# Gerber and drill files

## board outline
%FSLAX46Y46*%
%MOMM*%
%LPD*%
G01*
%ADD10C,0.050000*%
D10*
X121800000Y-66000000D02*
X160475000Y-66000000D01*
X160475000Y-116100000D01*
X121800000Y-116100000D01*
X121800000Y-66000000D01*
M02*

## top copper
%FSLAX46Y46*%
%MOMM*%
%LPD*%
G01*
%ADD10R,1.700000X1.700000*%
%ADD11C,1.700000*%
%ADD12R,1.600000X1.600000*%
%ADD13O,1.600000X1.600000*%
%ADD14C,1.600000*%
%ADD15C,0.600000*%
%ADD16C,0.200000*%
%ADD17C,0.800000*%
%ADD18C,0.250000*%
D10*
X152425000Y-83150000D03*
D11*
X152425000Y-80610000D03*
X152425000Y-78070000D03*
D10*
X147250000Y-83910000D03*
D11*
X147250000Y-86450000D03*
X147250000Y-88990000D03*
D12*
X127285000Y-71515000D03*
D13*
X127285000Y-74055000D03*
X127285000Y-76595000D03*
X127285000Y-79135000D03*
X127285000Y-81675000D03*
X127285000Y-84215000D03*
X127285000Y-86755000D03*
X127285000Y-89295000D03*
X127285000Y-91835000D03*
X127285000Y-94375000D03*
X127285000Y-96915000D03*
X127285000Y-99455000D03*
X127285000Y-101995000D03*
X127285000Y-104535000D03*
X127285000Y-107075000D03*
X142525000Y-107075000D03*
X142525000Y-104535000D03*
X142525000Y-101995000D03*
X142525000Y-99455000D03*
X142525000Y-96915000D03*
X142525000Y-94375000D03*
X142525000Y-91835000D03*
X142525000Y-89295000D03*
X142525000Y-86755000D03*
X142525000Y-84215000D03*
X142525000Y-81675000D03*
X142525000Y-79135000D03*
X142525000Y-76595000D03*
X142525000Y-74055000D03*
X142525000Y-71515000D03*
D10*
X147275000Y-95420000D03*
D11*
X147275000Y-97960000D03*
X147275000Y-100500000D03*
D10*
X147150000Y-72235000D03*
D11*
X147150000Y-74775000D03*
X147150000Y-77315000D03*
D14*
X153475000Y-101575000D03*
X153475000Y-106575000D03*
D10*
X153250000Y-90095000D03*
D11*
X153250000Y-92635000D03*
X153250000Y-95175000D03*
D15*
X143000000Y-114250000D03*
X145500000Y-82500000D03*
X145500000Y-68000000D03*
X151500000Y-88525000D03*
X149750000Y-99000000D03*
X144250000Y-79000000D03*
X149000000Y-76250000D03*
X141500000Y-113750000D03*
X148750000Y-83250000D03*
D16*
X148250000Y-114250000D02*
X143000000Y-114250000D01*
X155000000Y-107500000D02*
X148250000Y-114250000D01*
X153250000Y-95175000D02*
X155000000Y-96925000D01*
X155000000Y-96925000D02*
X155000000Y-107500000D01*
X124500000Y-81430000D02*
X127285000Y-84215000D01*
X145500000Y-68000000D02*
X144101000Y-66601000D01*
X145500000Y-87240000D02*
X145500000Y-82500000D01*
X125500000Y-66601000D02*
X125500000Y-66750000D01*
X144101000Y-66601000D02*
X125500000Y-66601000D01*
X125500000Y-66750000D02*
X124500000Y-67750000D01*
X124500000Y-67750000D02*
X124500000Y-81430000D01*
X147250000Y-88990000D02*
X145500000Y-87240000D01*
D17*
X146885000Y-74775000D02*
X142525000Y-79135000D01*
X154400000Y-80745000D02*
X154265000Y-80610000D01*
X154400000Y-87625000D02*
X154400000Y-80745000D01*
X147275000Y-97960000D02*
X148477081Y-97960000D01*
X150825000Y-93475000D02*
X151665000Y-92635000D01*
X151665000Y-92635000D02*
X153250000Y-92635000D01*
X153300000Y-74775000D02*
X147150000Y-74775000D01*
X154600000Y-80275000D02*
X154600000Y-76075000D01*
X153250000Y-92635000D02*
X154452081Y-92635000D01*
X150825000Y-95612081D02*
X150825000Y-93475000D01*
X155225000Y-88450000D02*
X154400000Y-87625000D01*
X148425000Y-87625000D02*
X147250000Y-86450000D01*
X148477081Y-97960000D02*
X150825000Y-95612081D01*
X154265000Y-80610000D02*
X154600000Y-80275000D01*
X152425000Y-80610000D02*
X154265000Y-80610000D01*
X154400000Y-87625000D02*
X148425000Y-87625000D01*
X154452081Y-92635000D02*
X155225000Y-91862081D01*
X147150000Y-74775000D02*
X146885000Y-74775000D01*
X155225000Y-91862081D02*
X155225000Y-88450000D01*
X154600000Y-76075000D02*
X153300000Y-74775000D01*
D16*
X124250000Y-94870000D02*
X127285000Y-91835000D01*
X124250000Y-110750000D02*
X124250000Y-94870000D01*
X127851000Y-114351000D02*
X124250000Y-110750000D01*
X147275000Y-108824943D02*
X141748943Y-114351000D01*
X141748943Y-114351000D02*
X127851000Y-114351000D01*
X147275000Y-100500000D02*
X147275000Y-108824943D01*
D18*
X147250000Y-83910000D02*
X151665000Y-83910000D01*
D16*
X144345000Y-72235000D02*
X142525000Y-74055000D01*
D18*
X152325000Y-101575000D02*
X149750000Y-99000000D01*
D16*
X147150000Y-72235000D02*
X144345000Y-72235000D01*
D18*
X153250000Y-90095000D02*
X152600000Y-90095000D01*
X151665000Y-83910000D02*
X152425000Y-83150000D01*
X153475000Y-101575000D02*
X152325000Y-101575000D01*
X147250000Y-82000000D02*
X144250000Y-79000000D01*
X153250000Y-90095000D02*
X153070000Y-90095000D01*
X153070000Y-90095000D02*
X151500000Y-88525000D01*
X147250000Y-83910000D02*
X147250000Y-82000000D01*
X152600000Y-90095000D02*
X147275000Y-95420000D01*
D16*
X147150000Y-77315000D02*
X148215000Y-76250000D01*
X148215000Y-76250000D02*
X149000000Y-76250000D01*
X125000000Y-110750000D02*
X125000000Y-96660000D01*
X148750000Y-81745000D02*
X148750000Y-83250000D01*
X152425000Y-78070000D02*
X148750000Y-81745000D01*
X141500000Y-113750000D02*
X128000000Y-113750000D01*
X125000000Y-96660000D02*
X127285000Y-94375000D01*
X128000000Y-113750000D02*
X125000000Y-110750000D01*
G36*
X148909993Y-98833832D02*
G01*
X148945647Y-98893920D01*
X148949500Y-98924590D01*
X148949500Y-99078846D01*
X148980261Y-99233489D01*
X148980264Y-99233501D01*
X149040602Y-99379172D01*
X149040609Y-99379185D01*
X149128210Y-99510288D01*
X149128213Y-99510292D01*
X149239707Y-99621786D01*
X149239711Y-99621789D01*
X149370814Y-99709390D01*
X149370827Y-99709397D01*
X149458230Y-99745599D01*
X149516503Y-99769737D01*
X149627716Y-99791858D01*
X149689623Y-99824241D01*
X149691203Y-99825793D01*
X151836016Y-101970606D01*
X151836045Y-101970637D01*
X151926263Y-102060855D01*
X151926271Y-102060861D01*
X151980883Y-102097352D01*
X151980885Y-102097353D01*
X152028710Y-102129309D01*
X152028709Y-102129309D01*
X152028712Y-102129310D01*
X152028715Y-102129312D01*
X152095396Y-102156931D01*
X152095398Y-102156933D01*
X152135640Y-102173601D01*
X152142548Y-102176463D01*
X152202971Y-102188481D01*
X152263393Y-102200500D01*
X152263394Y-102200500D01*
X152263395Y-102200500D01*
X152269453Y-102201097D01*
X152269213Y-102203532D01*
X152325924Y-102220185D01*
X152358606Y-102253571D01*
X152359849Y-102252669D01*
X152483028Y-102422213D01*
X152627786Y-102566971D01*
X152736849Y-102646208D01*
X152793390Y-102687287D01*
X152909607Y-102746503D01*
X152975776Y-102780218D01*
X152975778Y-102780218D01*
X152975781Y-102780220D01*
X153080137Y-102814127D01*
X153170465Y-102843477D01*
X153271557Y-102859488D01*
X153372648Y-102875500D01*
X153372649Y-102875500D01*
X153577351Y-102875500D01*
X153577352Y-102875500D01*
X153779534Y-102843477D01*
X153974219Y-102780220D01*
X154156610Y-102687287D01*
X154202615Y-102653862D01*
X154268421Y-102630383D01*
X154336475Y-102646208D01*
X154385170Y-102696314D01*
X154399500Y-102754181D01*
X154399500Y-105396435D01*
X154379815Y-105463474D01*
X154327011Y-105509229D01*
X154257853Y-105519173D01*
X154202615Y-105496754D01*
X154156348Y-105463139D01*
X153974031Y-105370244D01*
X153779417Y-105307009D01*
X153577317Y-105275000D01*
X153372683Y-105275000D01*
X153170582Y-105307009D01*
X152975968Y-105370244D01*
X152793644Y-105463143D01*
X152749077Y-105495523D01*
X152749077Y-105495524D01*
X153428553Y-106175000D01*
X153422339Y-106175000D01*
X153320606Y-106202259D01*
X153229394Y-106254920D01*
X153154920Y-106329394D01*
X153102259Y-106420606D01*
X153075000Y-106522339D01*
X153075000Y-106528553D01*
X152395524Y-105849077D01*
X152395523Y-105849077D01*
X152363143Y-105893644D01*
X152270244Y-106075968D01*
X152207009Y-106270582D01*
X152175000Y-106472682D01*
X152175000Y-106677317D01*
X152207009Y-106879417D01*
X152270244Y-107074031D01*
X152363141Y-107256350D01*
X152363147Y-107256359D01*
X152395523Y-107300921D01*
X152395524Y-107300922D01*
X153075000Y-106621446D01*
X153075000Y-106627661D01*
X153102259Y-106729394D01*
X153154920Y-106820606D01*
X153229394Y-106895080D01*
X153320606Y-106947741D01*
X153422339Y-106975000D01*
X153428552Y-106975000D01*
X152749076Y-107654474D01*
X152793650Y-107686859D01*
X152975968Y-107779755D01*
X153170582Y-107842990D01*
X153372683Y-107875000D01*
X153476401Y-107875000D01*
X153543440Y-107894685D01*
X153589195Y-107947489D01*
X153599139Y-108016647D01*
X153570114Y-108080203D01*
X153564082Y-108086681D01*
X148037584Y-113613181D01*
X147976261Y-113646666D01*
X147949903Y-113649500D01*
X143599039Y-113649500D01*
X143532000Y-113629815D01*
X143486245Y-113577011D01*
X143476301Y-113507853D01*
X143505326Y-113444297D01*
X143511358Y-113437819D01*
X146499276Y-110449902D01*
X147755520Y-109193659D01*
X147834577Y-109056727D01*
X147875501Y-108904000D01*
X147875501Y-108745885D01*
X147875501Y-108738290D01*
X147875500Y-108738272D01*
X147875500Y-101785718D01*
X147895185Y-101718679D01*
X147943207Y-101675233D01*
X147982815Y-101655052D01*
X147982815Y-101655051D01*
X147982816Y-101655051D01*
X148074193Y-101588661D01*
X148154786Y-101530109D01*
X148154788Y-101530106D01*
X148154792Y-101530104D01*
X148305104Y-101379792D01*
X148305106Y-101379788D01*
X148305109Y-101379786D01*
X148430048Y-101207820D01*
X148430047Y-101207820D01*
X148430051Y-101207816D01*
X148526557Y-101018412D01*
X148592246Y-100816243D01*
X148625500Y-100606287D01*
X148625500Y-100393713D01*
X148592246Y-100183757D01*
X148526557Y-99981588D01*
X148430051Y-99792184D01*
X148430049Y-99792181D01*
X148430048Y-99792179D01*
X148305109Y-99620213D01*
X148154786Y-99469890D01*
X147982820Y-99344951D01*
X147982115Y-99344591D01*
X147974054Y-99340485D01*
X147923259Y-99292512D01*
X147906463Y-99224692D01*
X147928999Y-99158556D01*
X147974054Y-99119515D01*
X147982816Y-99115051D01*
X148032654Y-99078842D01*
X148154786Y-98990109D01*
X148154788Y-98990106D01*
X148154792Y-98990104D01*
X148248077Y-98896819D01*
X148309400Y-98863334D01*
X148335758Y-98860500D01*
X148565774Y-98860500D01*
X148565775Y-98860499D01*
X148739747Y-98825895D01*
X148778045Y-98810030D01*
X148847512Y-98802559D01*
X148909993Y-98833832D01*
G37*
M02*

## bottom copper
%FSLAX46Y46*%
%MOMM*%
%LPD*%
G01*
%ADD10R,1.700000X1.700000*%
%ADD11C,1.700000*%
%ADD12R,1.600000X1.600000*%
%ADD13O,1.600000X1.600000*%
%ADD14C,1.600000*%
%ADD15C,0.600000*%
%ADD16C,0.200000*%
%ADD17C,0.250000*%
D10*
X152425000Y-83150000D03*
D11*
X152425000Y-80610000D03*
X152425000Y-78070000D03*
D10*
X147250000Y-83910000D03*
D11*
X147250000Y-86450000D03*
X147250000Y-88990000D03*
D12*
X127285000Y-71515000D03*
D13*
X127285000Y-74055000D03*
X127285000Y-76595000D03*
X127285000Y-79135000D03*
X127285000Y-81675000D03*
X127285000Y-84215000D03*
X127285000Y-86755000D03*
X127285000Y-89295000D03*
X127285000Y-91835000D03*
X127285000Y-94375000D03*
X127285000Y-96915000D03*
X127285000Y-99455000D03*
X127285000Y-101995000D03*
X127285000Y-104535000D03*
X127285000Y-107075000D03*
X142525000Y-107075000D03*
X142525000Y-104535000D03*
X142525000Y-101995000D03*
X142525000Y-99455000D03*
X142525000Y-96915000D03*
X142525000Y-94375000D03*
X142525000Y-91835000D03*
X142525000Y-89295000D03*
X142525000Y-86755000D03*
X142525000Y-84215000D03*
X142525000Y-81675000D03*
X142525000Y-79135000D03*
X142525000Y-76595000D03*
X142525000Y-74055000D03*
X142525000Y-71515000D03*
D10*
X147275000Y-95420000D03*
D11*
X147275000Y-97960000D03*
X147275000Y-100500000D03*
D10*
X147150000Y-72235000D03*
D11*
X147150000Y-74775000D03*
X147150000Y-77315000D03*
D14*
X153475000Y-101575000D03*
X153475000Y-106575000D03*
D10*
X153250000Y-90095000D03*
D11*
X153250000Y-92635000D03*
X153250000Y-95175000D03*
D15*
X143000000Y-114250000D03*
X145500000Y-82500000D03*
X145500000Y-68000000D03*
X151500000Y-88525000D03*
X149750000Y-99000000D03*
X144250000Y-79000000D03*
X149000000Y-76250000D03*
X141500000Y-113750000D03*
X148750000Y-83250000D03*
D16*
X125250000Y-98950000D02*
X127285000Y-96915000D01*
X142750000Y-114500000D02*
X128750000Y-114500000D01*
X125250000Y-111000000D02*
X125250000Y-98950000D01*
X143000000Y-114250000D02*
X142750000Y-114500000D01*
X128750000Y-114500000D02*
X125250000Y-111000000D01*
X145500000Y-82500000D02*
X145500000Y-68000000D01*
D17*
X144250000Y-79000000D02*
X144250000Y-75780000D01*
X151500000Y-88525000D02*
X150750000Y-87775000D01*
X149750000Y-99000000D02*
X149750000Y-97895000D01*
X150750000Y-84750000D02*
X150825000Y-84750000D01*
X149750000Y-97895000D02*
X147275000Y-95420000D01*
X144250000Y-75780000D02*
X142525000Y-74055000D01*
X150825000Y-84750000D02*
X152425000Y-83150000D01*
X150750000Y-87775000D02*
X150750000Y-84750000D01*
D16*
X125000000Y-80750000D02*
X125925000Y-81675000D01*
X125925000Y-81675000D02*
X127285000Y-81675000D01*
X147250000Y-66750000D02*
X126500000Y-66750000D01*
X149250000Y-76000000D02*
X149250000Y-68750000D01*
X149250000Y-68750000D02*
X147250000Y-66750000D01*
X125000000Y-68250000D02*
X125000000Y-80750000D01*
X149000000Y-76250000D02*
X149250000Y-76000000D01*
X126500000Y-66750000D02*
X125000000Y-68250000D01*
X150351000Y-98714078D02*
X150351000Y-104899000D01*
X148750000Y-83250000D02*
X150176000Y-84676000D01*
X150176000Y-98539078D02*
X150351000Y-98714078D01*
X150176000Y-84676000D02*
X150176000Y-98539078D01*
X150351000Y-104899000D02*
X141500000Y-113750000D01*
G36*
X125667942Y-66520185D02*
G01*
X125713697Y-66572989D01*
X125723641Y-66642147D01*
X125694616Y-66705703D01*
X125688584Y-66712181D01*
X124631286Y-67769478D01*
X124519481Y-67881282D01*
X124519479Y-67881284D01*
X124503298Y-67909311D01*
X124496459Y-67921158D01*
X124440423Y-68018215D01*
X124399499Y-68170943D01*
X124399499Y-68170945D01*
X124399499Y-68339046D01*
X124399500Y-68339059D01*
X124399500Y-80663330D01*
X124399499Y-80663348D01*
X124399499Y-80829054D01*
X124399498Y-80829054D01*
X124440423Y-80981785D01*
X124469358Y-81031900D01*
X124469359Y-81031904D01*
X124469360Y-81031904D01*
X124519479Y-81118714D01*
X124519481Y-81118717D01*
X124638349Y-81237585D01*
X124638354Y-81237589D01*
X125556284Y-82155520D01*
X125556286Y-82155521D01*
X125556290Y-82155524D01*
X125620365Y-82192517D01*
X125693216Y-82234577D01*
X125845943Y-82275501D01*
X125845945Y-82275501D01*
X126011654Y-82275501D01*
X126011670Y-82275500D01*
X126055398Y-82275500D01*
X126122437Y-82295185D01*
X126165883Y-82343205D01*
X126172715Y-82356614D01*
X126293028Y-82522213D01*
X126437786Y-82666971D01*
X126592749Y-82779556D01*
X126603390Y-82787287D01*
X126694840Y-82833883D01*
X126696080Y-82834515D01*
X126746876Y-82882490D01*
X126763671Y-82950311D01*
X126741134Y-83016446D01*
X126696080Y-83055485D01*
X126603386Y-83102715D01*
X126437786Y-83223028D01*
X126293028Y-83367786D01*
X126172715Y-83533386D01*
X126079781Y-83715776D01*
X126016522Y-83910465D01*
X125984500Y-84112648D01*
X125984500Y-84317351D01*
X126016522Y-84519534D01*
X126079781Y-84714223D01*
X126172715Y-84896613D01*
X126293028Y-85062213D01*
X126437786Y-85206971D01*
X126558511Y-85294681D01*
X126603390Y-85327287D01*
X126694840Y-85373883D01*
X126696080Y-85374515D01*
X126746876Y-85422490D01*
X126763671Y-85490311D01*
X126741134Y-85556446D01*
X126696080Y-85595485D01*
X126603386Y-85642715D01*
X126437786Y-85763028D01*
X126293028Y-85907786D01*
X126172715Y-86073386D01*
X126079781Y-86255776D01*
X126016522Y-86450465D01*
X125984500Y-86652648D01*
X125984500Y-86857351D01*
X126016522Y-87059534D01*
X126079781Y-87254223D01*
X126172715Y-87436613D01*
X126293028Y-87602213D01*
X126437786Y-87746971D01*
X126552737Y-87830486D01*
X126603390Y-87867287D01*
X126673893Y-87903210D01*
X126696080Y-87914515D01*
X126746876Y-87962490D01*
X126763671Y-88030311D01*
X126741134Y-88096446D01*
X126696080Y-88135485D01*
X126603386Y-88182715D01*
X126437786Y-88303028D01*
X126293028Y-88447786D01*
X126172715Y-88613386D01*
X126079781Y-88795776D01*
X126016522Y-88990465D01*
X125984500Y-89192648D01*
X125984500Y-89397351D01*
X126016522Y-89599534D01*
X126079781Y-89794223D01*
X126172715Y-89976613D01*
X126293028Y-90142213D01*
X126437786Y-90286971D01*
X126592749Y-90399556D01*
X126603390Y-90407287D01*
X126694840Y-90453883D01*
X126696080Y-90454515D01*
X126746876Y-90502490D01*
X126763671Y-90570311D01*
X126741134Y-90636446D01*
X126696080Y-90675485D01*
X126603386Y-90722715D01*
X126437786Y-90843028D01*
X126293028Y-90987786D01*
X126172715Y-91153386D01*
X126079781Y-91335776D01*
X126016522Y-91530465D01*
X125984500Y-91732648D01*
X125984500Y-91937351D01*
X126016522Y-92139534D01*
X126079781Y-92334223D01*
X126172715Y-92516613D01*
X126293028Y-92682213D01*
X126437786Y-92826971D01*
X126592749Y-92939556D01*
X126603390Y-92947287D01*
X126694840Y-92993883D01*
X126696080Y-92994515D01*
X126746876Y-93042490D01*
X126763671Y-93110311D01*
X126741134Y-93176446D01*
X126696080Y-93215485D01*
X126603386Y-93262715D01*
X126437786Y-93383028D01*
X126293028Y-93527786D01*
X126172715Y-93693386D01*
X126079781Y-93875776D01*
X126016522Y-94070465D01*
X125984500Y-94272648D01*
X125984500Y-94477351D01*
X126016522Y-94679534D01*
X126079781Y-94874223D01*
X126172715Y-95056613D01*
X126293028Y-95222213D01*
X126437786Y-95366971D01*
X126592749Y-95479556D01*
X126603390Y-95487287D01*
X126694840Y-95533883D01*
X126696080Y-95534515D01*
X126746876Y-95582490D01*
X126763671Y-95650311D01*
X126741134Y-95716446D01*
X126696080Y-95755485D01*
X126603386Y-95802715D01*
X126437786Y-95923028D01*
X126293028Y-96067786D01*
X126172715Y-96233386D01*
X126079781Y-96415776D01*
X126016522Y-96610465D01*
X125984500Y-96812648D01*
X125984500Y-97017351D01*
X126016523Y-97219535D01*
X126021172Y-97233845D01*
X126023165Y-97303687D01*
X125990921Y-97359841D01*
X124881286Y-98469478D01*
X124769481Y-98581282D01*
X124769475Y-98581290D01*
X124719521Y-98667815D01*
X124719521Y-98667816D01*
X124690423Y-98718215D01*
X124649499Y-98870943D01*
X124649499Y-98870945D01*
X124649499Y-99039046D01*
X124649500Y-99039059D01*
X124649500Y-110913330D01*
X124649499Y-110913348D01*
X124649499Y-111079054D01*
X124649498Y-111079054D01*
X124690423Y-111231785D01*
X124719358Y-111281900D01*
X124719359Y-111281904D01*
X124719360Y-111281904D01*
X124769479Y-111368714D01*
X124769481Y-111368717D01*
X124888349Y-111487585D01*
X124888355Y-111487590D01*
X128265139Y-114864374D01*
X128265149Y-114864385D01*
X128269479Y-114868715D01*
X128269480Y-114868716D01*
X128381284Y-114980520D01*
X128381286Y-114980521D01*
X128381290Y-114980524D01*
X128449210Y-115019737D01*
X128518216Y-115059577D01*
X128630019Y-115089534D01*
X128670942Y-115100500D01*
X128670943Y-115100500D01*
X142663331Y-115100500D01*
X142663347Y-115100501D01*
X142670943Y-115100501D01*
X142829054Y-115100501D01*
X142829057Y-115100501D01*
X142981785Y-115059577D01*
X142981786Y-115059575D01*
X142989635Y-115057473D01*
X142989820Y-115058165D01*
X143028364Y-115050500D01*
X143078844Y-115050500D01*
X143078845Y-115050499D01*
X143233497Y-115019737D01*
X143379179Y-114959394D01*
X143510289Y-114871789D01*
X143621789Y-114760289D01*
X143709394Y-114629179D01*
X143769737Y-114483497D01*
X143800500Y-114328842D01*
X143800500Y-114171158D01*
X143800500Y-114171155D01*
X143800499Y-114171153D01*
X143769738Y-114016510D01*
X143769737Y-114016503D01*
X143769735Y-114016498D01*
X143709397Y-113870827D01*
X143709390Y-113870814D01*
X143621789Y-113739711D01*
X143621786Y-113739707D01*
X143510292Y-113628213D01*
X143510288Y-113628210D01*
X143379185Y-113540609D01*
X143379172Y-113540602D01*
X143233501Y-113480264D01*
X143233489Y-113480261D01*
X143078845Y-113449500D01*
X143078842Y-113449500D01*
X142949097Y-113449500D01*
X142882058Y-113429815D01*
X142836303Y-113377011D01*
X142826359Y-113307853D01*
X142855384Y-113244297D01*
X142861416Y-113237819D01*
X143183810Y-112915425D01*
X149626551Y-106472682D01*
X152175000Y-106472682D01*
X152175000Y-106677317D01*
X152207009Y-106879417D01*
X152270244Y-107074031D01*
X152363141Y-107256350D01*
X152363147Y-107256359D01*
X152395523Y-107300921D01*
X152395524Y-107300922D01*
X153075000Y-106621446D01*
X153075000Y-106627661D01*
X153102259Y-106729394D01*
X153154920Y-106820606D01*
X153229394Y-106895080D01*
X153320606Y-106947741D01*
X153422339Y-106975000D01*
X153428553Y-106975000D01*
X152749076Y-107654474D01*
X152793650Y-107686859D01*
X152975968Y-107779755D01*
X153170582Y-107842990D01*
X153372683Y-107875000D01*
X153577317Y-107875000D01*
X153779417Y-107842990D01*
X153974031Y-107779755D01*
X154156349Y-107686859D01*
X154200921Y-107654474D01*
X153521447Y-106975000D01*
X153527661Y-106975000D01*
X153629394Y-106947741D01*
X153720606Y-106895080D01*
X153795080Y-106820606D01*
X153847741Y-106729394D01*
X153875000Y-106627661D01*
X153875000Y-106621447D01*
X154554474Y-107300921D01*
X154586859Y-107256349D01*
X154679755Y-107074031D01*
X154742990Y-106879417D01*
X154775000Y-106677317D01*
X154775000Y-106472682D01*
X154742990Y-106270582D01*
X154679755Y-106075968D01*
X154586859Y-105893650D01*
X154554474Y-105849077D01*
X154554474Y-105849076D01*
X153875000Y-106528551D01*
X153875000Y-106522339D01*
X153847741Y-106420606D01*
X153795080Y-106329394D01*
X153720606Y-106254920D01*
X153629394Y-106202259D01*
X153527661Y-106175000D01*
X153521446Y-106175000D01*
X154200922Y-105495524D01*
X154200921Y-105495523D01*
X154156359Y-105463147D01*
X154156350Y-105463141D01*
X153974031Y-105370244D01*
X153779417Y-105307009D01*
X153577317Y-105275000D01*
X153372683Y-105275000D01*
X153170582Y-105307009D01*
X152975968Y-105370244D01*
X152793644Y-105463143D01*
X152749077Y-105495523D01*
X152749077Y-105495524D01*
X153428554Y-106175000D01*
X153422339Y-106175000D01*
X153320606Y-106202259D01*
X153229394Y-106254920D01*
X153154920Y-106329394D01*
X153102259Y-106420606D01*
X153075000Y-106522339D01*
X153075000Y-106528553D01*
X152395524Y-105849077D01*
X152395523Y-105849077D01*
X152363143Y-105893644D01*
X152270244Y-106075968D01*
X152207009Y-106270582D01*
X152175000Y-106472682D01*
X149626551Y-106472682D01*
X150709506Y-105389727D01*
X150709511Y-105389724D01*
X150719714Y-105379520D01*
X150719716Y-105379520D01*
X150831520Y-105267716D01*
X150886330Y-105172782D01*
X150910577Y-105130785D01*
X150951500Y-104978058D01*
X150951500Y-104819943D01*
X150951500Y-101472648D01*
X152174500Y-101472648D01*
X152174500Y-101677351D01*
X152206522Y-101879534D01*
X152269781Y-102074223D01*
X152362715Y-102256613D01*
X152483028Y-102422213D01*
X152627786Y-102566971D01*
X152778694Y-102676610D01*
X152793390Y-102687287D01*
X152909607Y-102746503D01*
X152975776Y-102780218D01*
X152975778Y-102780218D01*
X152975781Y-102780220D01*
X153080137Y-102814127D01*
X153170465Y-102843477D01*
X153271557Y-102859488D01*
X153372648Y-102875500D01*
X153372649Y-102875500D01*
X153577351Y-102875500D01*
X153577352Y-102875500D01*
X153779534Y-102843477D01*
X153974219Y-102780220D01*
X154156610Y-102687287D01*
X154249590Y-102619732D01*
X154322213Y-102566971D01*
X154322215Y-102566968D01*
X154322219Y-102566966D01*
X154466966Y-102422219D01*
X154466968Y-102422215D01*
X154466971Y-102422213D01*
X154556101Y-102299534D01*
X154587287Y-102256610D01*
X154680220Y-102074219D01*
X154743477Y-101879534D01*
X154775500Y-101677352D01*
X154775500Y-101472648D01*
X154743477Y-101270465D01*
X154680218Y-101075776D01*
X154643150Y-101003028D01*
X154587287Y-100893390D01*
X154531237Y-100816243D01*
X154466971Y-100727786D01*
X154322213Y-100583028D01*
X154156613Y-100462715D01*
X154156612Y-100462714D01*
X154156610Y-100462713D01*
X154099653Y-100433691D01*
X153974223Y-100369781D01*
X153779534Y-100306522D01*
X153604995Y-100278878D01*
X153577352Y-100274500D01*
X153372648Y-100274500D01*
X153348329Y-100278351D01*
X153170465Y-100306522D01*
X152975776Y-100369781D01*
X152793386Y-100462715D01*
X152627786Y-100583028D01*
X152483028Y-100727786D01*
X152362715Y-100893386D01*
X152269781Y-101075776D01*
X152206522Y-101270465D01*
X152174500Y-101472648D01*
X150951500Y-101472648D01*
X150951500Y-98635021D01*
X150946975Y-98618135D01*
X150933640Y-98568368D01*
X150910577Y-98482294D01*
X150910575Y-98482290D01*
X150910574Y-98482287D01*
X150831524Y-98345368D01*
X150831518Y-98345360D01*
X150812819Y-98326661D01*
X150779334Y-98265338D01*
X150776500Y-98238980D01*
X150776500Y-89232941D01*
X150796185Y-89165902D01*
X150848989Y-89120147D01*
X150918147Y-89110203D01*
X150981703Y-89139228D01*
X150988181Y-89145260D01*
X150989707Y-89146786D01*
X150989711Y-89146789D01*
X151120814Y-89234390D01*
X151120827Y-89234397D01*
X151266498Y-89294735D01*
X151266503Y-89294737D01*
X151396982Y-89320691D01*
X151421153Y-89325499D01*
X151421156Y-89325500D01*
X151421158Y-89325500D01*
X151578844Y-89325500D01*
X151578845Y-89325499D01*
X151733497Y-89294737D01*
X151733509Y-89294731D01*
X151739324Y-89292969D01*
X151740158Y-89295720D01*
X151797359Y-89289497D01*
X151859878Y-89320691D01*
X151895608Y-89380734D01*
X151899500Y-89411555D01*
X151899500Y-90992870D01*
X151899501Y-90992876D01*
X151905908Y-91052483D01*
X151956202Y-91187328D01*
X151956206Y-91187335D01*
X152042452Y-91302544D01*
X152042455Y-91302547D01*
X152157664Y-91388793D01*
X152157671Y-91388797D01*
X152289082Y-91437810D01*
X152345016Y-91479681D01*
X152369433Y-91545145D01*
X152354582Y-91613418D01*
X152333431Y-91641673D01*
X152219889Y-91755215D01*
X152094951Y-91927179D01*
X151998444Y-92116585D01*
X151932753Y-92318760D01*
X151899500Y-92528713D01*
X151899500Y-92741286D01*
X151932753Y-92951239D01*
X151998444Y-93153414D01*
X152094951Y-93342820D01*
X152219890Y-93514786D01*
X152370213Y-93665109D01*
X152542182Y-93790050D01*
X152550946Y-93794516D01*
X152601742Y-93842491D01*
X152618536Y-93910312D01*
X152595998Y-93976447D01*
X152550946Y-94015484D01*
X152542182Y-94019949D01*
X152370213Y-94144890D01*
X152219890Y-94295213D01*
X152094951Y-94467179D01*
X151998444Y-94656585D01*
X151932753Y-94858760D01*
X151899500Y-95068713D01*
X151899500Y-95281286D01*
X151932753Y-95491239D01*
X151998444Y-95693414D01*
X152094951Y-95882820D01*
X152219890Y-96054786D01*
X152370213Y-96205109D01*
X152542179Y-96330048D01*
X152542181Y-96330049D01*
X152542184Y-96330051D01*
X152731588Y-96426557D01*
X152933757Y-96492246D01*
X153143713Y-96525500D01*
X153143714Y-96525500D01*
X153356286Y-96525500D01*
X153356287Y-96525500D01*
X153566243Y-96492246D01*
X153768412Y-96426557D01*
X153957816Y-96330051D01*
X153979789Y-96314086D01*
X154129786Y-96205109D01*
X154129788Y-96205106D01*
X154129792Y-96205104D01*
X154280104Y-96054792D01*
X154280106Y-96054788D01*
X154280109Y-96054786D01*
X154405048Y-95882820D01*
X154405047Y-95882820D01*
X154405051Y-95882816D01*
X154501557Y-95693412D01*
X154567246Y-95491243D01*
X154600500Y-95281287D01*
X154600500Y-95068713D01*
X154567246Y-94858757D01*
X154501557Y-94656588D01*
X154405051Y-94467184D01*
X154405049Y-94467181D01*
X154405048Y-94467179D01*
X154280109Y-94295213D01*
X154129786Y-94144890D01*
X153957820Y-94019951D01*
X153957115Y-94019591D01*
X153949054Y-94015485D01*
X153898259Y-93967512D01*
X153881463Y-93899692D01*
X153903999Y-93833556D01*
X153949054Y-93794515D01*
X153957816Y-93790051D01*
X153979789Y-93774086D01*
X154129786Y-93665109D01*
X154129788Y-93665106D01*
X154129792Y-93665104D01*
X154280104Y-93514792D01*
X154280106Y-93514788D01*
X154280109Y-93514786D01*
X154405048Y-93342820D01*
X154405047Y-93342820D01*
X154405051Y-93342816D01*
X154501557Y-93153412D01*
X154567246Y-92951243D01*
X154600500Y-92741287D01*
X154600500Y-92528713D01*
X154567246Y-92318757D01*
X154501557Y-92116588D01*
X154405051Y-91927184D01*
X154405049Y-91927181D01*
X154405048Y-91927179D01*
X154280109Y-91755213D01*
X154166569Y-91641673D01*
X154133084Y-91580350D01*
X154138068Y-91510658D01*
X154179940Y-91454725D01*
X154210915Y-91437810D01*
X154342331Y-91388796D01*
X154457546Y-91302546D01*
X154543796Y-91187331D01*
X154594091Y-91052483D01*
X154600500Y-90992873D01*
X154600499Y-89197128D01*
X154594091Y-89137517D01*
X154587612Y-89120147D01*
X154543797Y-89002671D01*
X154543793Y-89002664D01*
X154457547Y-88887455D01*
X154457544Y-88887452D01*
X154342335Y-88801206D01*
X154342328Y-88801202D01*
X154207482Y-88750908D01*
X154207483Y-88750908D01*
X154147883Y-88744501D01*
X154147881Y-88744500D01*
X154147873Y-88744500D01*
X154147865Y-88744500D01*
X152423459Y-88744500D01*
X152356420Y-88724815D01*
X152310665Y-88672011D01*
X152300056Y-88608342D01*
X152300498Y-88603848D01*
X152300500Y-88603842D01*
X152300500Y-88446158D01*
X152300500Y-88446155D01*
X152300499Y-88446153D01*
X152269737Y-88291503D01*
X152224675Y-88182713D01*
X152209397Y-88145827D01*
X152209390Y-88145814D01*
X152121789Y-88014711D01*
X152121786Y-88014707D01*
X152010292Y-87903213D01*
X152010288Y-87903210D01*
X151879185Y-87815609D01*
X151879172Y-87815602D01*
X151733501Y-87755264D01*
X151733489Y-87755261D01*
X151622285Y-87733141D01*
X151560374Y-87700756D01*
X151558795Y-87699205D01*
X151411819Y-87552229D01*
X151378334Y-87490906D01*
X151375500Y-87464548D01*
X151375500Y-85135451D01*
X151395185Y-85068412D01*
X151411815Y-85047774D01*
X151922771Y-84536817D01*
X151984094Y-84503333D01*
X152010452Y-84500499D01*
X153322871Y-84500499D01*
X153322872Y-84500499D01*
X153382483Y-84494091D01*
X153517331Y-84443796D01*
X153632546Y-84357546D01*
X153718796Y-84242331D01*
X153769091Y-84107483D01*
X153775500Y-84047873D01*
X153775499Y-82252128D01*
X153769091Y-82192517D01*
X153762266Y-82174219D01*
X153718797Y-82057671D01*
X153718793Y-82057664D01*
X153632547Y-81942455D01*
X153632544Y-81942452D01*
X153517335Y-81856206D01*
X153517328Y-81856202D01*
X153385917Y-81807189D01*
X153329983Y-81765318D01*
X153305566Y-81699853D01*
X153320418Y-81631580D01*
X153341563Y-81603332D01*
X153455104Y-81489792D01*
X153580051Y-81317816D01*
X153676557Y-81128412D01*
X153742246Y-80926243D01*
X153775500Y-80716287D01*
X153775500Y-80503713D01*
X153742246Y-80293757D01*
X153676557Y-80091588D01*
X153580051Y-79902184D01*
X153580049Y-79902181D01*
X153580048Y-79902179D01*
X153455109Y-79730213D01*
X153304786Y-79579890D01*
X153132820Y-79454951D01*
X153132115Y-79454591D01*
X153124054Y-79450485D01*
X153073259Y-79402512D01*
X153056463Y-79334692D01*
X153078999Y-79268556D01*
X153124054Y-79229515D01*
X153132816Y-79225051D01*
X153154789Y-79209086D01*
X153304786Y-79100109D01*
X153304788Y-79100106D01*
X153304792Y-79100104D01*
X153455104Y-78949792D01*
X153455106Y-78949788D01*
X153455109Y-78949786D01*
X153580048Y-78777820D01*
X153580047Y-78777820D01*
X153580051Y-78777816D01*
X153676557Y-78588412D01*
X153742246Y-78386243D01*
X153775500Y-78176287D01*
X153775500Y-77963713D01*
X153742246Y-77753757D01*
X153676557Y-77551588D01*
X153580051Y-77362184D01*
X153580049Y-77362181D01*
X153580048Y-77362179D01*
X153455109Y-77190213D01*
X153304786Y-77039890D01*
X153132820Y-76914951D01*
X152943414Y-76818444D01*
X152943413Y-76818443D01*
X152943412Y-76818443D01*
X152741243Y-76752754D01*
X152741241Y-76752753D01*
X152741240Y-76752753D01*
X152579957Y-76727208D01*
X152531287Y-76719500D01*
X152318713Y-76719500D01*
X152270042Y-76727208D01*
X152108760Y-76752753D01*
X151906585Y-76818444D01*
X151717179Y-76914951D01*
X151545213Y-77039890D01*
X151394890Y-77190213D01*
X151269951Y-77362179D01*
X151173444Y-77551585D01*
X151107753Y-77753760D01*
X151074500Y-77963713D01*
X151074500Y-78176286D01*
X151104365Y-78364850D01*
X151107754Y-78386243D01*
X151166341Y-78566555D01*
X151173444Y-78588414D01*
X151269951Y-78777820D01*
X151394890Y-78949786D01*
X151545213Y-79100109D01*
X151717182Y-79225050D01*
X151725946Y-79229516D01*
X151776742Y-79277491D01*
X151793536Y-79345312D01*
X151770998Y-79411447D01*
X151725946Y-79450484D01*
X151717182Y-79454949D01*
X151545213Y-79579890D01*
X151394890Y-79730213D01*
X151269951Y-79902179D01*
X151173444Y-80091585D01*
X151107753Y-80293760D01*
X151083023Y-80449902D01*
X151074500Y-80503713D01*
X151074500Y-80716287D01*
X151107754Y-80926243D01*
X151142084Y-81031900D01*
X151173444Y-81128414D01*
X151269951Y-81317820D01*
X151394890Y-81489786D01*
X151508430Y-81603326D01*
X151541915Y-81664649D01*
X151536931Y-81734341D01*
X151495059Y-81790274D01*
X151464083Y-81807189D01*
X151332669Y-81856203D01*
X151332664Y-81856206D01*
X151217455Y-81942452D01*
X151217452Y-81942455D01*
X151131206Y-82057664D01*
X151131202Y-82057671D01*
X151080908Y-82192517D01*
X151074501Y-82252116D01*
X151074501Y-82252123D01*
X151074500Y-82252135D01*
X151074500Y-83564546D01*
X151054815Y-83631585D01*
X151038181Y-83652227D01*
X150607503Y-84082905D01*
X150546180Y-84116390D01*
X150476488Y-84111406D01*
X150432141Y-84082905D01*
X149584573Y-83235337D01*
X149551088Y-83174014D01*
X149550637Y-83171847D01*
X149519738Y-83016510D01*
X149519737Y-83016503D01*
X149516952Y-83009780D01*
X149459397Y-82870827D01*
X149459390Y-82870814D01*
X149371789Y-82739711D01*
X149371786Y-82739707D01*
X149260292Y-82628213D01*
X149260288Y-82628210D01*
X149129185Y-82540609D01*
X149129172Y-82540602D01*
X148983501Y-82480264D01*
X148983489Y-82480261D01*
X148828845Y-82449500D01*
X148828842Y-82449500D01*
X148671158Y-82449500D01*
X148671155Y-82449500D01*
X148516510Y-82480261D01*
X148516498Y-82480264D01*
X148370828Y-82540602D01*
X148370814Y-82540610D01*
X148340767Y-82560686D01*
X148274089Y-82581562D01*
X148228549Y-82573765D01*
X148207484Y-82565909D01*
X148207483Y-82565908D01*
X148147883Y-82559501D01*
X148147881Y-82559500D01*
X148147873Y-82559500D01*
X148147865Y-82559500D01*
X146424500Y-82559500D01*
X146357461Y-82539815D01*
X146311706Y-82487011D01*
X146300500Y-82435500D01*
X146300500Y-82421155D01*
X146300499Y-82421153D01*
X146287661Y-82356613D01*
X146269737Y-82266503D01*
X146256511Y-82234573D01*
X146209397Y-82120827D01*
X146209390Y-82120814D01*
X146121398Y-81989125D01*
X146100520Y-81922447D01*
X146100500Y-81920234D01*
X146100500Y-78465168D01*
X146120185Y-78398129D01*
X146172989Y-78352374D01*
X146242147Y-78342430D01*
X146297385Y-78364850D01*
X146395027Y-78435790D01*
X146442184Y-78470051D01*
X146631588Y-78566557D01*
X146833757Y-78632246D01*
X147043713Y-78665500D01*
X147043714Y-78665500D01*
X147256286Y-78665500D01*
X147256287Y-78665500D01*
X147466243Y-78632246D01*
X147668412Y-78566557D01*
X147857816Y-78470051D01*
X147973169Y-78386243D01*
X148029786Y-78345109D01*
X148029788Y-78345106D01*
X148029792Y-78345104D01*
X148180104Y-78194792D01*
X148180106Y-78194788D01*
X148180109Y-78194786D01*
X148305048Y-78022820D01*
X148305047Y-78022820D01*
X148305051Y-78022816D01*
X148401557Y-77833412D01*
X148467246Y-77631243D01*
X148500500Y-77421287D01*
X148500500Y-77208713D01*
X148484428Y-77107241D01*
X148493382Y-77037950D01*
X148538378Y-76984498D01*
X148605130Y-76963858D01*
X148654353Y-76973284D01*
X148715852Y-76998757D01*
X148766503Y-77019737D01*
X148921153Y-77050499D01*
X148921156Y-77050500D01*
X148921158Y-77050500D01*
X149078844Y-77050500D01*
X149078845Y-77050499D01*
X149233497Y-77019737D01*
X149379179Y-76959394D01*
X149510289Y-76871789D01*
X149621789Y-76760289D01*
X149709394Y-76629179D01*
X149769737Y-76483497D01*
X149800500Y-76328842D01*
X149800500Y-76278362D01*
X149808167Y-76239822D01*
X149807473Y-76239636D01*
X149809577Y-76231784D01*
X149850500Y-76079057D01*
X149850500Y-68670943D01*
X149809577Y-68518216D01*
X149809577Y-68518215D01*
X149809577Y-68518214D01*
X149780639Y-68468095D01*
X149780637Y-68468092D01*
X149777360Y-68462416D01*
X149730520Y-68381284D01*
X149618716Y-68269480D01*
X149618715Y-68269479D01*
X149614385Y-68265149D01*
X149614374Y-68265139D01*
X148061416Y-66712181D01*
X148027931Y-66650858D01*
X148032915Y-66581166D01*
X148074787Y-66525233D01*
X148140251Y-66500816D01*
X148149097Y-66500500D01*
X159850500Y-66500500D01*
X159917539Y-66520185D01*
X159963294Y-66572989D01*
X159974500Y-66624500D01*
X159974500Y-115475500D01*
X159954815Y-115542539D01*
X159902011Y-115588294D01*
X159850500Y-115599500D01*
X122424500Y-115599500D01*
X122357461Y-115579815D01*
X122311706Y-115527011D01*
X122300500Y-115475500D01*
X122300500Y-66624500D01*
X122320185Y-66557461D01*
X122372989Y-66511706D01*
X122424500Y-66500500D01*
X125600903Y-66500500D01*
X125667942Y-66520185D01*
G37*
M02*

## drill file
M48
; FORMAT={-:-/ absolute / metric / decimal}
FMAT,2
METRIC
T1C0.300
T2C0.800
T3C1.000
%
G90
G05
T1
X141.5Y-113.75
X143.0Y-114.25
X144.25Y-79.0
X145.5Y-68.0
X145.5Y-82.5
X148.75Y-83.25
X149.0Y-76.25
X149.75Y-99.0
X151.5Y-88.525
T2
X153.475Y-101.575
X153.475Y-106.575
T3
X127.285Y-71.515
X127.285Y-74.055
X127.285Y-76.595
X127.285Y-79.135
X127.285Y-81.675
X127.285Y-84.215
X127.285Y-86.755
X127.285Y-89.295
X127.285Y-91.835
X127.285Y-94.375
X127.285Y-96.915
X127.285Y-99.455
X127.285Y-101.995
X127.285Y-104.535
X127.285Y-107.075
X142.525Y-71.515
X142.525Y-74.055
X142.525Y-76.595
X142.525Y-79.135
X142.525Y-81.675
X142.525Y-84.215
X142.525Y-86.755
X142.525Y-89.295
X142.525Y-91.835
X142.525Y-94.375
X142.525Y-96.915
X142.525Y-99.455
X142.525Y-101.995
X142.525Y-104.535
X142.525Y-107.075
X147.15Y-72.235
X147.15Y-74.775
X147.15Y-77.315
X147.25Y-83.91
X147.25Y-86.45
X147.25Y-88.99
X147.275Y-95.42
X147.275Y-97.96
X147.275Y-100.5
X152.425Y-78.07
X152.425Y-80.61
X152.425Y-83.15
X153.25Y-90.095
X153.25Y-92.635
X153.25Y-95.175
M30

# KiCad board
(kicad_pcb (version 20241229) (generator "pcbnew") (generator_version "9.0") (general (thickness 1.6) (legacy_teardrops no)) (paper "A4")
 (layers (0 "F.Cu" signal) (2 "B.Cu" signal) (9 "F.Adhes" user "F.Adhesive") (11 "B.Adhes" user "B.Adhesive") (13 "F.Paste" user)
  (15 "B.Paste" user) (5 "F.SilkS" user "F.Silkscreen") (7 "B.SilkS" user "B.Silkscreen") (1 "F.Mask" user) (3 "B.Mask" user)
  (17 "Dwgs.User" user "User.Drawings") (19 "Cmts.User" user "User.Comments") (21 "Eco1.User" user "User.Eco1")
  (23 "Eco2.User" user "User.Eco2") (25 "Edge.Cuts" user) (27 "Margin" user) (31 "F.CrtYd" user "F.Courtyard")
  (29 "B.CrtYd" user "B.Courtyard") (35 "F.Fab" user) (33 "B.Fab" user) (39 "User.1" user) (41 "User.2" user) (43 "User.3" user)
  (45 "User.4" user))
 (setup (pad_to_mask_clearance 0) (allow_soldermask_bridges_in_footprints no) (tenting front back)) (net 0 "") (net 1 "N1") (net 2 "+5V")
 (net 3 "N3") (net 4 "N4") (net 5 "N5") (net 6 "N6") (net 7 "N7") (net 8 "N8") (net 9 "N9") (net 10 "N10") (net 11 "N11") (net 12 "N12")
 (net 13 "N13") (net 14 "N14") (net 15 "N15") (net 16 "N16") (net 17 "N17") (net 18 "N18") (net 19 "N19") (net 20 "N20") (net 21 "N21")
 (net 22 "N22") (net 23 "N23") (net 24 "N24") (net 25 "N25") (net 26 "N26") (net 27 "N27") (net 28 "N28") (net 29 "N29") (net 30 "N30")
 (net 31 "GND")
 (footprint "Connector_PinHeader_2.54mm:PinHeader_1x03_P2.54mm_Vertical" (layer "F.Cu") (at 152.425 83.15 180)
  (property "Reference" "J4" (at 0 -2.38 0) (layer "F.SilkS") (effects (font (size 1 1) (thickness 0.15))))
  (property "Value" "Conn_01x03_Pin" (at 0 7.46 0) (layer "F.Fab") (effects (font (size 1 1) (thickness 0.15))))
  (pad "1" thru_hole rect (at 0 0 180) (size 1.7 1.7) (drill 1) (layers "*.Cu" "*.Mask") (remove_unused_layers no) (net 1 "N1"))
  (pad "2" thru_hole circle (at 0 2.54 180) (size 1.7 1.7) (drill 1) (layers "*.Cu" "*.Mask") (remove_unused_layers no) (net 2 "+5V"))
  (pad "3" thru_hole circle (at 0 5.08 180) (size 1.7 1.7) (drill 1) (layers "*.Cu" "*.Mask") (remove_unused_layers no) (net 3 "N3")))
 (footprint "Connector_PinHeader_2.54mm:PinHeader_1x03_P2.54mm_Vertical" (layer "F.Cu") (at 147.25 83.91)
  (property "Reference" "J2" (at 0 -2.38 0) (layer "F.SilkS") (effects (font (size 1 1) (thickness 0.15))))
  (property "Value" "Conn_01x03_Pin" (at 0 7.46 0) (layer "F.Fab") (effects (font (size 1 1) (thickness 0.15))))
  (pad "1" thru_hole rect (at 0 0) (size 1.7 1.7) (drill 1) (layers "*.Cu" "*.Mask") (remove_unused_layers no) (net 1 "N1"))
  (pad "2" thru_hole circle (at 0 2.54) (size 1.7 1.7) (drill 1) (layers "*.Cu" "*.Mask") (remove_unused_layers no) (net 2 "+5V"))
  (pad "3" thru_hole circle (at 0 5.08) (size 1.7 1.7) (drill 1) (layers "*.Cu" "*.Mask") (remove_unused_layers no) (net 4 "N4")))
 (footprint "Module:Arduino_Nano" (layer "F.Cu") (at 127.285 71.515)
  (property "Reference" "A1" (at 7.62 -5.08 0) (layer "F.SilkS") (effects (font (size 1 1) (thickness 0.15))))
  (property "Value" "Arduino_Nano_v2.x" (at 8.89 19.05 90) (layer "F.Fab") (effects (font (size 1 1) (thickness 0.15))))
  (pad "1" thru_hole rect (at 0 0) (size 1.6 1.6) (drill 1) (layers "*.Cu" "*.Mask") (remove_unused_layers no) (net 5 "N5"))
  (pad "2" thru_hole oval (at 0 2.54) (size 1.6 1.6) (drill 1) (layers "*.Cu" "*.Mask") (remove_unused_layers no) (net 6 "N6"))
  (pad "3" thru_hole oval (at 0 5.08) (size 1.6 1.6) (drill 1) (layers "*.Cu" "*.Mask") (remove_unused_layers no) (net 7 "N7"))
  (pad "4" thru_hole oval (at 0 7.62) (size 1.6 1.6) (drill 1) (layers "*.Cu" "*.Mask") (remove_unused_layers no) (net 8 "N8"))
  (pad "5" thru_hole oval (at 0 10.16) (size 1.6 1.6) (drill 1) (layers "*.Cu" "*.Mask") (remove_unused_layers no) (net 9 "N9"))
  (pad "6" thru_hole oval (at 0 12.7) (size 1.6 1.6) (drill 1) (layers "*.Cu" "*.Mask") (remove_unused_layers no) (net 4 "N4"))
  (pad "7" thru_hole oval (at 0 15.24) (size 1.6 1.6) (drill 1) (layers "*.Cu" "*.Mask") (remove_unused_layers no) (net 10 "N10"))
  (pad "8" thru_hole oval (at 0 17.78) (size 1.6 1.6) (drill 1) (layers "*.Cu" "*.Mask") (remove_unused_layers no) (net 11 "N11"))
  (pad "9" thru_hole oval (at 0 20.32) (size 1.6 1.6) (drill 1) (layers "*.Cu" "*.Mask") (remove_unused_layers no) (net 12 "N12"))
  (pad "10" thru_hole oval (at 0 22.86) (size 1.6 1.6) (drill 1) (layers "*.Cu" "*.Mask") (remove_unused_layers no) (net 3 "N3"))
  (pad "11" thru_hole oval (at 0 25.4) (size 1.6 1.6) (drill 1) (layers "*.Cu" "*.Mask") (remove_unused_layers no) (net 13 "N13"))
  (pad "12" thru_hole oval (at 0 27.94) (size 1.6 1.6) (drill 1) (layers "*.Cu" "*.Mask") (remove_unused_layers no) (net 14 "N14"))
  (pad "13" thru_hole oval (at 0 30.48) (size 1.6 1.6) (drill 1) (layers "*.Cu" "*.Mask") (remove_unused_layers no) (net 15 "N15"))
  (pad "14" thru_hole oval (at 0 33.02) (size 1.6 1.6) (drill 1) (layers "*.Cu" "*.Mask") (remove_unused_layers no) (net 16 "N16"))
  (pad "15" thru_hole oval (at 0 35.56) (size 1.6 1.6) (drill 1) (layers "*.Cu" "*.Mask") (remove_unused_layers no) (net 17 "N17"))
  (pad "16" thru_hole oval (at 15.24 35.56) (size 1.6 1.6) (drill 1) (layers "*.Cu" "*.Mask") (remove_unused_layers no) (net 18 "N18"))
  (pad "17" thru_hole oval (at 15.24 33.02) (size 1.6 1.6) (drill 1) (layers "*.Cu" "*.Mask") (remove_unused_layers no) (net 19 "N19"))
  (pad "18" thru_hole oval (at 15.24 30.48) (size 1.6 1.6) (drill 1) (layers "*.Cu" "*.Mask") (remove_unused_layers no) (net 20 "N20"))
  (pad "19" thru_hole oval (at 15.24 27.94) (size 1.6 1.6) (drill 1) (layers "*.Cu" "*.Mask") (remove_unused_layers no) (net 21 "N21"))
  (pad "20" thru_hole oval (at 15.24 25.4) (size 1.6 1.6) (drill 1) (layers "*.Cu" "*.Mask") (remove_unused_layers no) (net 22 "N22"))
  (pad "21" thru_hole oval (at 15.24 22.86) (size 1.6 1.6) (drill 1) (layers "*.Cu" "*.Mask") (remove_unused_layers no) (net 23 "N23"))
  (pad "22" thru_hole oval (at 15.24 20.32) (size 1.6 1.6) (drill 1) (layers "*.Cu" "*.Mask") (remove_unused_layers no) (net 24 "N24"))
  (pad "23" thru_hole oval (at 15.24 17.78) (size 1.6 1.6) (drill 1) (layers "*.Cu" "*.Mask") (remove_unused_layers no) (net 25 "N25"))
  (pad "24" thru_hole oval (at 15.24 15.24) (size 1.6 1.6) (drill 1) (layers "*.Cu" "*.Mask") (remove_unused_layers no) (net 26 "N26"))
  (pad "25" thru_hole oval (at 15.24 12.7) (size 1.6 1.6) (drill 1) (layers "*.Cu" "*.Mask") (remove_unused_layers no) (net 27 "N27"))
  (pad "26" thru_hole oval (at 15.24 10.16) (size 1.6 1.6) (drill 1) (layers "*.Cu" "*.Mask") (remove_unused_layers no) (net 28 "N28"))
  (pad "27" thru_hole oval (at 15.24 7.62) (size 1.6 1.6) (drill 1) (layers "*.Cu" "*.Mask") (remove_unused_layers no) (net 2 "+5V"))
  (pad "28" thru_hole oval (at 15.24 5.08) (size 1.6 1.6) (drill 1) (layers "*.Cu" "*.Mask") (remove_unused_layers no) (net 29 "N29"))
  (pad "29" thru_hole oval (at 15.24 2.54) (size 1.6 1.6) (drill 1) (layers "*.Cu" "*.Mask") (remove_unused_layers no) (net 1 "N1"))
  (pad "30" thru_hole oval (at 15.24 0) (size 1.6 1.6) (drill 1) (layers "*.Cu" "*.Mask") (remove_unused_layers no) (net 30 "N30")))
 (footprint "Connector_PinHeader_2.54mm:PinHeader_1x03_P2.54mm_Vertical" (layer "F.Cu") (at 147.275 95.42)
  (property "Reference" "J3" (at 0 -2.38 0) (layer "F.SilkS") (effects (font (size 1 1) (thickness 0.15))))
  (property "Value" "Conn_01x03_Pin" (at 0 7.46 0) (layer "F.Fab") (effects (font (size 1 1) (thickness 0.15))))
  (pad "1" thru_hole rect (at 0 0) (size 1.7 1.7) (drill 1) (layers "*.Cu" "*.Mask") (remove_unused_layers no) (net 1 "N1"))
  (pad "2" thru_hole circle (at 0 2.54) (size 1.7 1.7) (drill 1) (layers "*.Cu" "*.Mask") (remove_unused_layers no) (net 2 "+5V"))
  (pad "3" thru_hole circle (at 0 5.08) (size 1.7 1.7) (drill 1) (layers "*.Cu" "*.Mask") (remove_unused_layers no) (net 12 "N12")))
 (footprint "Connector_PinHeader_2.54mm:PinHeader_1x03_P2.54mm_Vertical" (layer "F.Cu") (at 147.15 72.235)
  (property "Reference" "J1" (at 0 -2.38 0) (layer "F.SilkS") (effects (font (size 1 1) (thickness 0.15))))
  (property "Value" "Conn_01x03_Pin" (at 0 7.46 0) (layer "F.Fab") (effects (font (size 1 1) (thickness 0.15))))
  (pad "1" thru_hole rect (at 0 0) (size 1.7 1.7) (drill 1) (layers "*.Cu" "*.Mask") (remove_unused_layers no) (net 1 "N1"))
  (pad "2" thru_hole circle (at 0 2.54) (size 1.7 1.7) (drill 1) (layers "*.Cu" "*.Mask") (remove_unused_layers no) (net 2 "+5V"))
  (pad "3" thru_hole circle (at 0 5.08) (size 1.7 1.7) (drill 1) (layers "*.Cu" "*.Mask") (remove_unused_layers no) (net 9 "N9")))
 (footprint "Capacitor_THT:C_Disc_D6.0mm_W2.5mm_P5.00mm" (layer "F.Cu") (at 153.475 101.575 -90)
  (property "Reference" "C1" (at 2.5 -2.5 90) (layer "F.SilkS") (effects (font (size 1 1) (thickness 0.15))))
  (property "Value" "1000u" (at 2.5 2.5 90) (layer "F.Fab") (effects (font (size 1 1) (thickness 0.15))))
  (pad "1" thru_hole circle (at 0 0 270) (size 1.6 1.6) (drill 0.8) (layers "*.Cu" "*.Mask") (remove_unused_layers no) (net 1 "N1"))
  (pad "2" thru_hole circle (at 5 0 270) (size 1.6 1.6) (drill 0.8) (layers "*.Cu" "*.Mask") (remove_unused_layers no) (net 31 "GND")))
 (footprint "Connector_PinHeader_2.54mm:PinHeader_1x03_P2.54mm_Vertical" (layer "F.Cu") (at 153.25 90.095)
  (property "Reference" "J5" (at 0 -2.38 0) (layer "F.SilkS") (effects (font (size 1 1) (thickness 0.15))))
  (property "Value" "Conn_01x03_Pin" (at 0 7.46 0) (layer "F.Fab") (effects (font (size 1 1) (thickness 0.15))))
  (pad "1" thru_hole rect (at 0 0) (size 1.7 1.7) (drill 1) (layers "*.Cu" "*.Mask") (remove_unused_layers no) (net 1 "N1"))
  (pad "2" thru_hole circle (at 0 2.54) (size 1.7 1.7) (drill 1) (layers "*.Cu" "*.Mask") (remove_unused_layers no) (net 2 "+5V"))
  (pad "3" thru_hole circle (at 0 5.08) (size 1.7 1.7) (drill 1) (layers "*.Cu" "*.Mask") (remove_unused_layers no) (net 13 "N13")))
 (gr_rect (start 121.8 66) (end 160.475 116.1) (stroke (width 0.05) (type default)) (fill no) (layer "Edge.Cuts"))
 (segment (start 148.25 114.25) (end 143 114.25) (width 0.2) (layer "F.Cu") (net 13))
 (segment (start 155 107.5) (end 148.25 114.25) (width 0.2) (layer "F.Cu") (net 13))
 (segment (start 153.25 95.175) (end 155 96.925) (width 0.2) (layer "F.Cu") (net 13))
 (segment (start 155 96.925) (end 155 107.5) (width 0.2) (layer "F.Cu") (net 13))
 (via (at 143 114.25) (size 0.6) (drill 0.3) (layers "F.Cu" "B.Cu") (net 13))
 (segment (start 125.25 98.95) (end 127.285 96.915) (width 0.2) (layer "B.Cu") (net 13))
 (segment (start 142.75 114.5) (end 128.75 114.5) (width 0.2) (layer "B.Cu") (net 13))
 (segment (start 125.25 111) (end 125.25 98.95) (width 0.2) (layer "B.Cu") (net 13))
 (segment (start 143 114.25) (end 142.75 114.5) (width 0.2) (layer "B.Cu") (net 13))
 (segment (start 128.75 114.5) (end 125.25 111) (width 0.2) (layer "B.Cu") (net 13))
 (segment (start 124.5 81.43) (end 127.285 84.215) (width 0.2) (layer "F.Cu") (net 4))
 (segment (start 145.5 68) (end 144.101 66.601) (width 0.2) (layer "F.Cu") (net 4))
 (segment (start 145.5 87.24) (end 145.5 82.5) (width 0.2) (layer "F.Cu") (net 4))
 (segment (start 125.5 66.601) (end 125.5 66.75) (width 0.2) (layer "F.Cu") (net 4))
 (segment (start 144.101 66.601) (end 125.5 66.601) (width 0.2) (layer "F.Cu") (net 4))
 (segment (start 125.5 66.75) (end 124.5 67.75) (width 0.2) (layer "F.Cu") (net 4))
 (segment (start 124.5 67.75) (end 124.5 81.43) (width 0.2) (layer "F.Cu") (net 4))
 (segment (start 147.25 88.99) (end 145.5 87.24) (width 0.2) (layer "F.Cu") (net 4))
 (via (at 145.5 82.5) (size 0.6) (drill 0.3) (layers "F.Cu" "B.Cu") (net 4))
 (via (at 145.5 68) (size 0.6) (drill 0.3) (layers "F.Cu" "B.Cu") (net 4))
 (segment (start 145.5 82.5) (end 145.5 68) (width 0.2) (layer "B.Cu") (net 4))
 (segment (start 146.885 74.775) (end 142.525 79.135) (width 0.8) (layer "F.Cu") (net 2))
 (segment (start 154.4 80.745) (end 154.265 80.61) (width 0.8) (layer "F.Cu") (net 2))
 (segment (start 154.4 87.625) (end 154.4 80.745) (width 0.8) (layer "F.Cu") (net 2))
 (segment (start 147.275 97.96) (end 148.477081 97.96) (width 0.8) (layer "F.Cu") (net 2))
 (segment (start 150.825 93.475) (end 151.665 92.635) (width 0.8) (layer "F.Cu") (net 2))
 (segment (start 151.665 92.635) (end 153.25 92.635) (width 0.8) (layer "F.Cu") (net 2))
 (segment (start 153.3 74.775) (end 147.15 74.775) (width 0.8) (layer "F.Cu") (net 2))
 (segment (start 154.6 80.275) (end 154.6 76.075) (width 0.8) (layer "F.Cu") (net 2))
 (segment (start 153.25 92.635) (end 154.452081 92.635) (width 0.8) (layer "F.Cu") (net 2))
 (segment (start 150.825 95.612081) (end 150.825 93.475) (width 0.8) (layer "F.Cu") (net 2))
 (segment (start 155.225 88.45) (end 154.4 87.625) (width 0.8) (layer "F.Cu") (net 2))
 (segment (start 148.425 87.625) (end 147.25 86.45) (width 0.8) (layer "F.Cu") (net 2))
 (segment (start 148.477081 97.96) (end 150.825 95.612081) (width 0.8) (layer "F.Cu") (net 2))
 (segment (start 154.265 80.61) (end 154.6 80.275) (width 0.8) (layer "F.Cu") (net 2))
 (segment (start 152.425 80.61) (end 154.265 80.61) (width 0.8) (layer "F.Cu") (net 2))
 (segment (start 154.4 87.625) (end 148.425 87.625) (width 0.8) (layer "F.Cu") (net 2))
 (segment (start 154.452081 92.635) (end 155.225 91.862081) (width 0.8) (layer "F.Cu") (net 2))
 (segment (start 147.15 74.775) (end 146.885 74.775) (width 0.8) (layer "F.Cu") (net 2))
 (segment (start 155.225 91.862081) (end 155.225 88.45) (width 0.8) (layer "F.Cu") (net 2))
 (segment (start 154.6 76.075) (end 153.3 74.775) (width 0.8) (layer "F.Cu") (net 2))
 (segment (start 124.25 94.87) (end 127.285 91.835) (width 0.2) (layer "F.Cu") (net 12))
 (segment (start 124.25 110.75) (end 124.25 94.87) (width 0.2) (layer "F.Cu") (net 12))
 (segment (start 127.851 114.351) (end 124.25 110.75) (width 0.2) (layer "F.Cu") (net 12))
 (segment (start 147.275 108.824943) (end 141.748943 114.351) (width 0.2) (layer "F.Cu") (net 12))
 (segment (start 141.748943 114.351) (end 127.851 114.351) (width 0.2) (layer "F.Cu") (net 12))
 (segment (start 147.275 100.5) (end 147.275 108.824943) (width 0.2) (layer "F.Cu") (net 12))
 (segment (start 147.25 83.91) (end 151.665 83.91) (width 0.25) (layer "F.Cu") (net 1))
 (segment (start 144.345 72.235) (end 142.525 74.055) (width 0.2) (layer "F.Cu") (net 1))
 (segment (start 152.325 101.575) (end 149.75 99) (width 0.25) (layer "F.Cu") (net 1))
 (segment (start 147.15 72.235) (end 144.345 72.235) (width 0.2) (layer "F.Cu") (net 1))
 (segment (start 153.25 90.095) (end 152.6 90.095) (width 0.25) (layer "F.Cu") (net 1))
 (segment (start 151.665 83.91) (end 152.425 83.15) (width 0.25) (layer "F.Cu") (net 1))
 (segment (start 153.475 101.575) (end 152.325 101.575) (width 0.25) (layer "F.Cu") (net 1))
 (segment (start 147.25 82) (end 144.25 79) (width 0.25) (layer "F.Cu") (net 1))
 (segment (start 153.25 90.095) (end 153.07 90.095) (width 0.25) (layer "F.Cu") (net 1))
 (segment (start 153.07 90.095) (end 151.5 88.525) (width 0.25) (layer "F.Cu") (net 1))
 (segment (start 147.25 83.91) (end 147.25 82) (width 0.25) (layer "F.Cu") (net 1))
 (segment (start 152.6 90.095) (end 147.275 95.42) (width 0.25) (layer "F.Cu") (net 1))
 (via (at 151.5 88.525) (size 0.6) (drill 0.3) (layers "F.Cu" "B.Cu") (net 1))
 (via (at 149.75 99) (size 0.6) (drill 0.3) (layers "F.Cu" "B.Cu") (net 1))
 (via (at 144.25 79) (size 0.6) (drill 0.3) (layers "F.Cu" "B.Cu") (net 1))
 (segment (start 144.25 79) (end 144.25 75.78) (width 0.25) (layer "B.Cu") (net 1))
 (segment (start 151.5 88.525) (end 150.75 87.775) (width 0.25) (layer "B.Cu") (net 1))
 (segment (start 149.75 99) (end 149.75 97.895) (width 0.25) (layer "B.Cu") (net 1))
 (segment (start 150.75 84.75) (end 150.825 84.75) (width 0.25) (layer "B.Cu") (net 1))
 (segment (start 149.75 97.895) (end 147.275 95.42) (width 0.25) (layer "B.Cu") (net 1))
 (segment (start 144.25 75.78) (end 142.525 74.055) (width 0.25) (layer "B.Cu") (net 1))
 (segment (start 150.825 84.75) (end 152.425 83.15) (width 0.25) (layer "B.Cu") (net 1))
 (segment (start 150.75 87.775) (end 150.75 84.75) (width 0.25) (layer "B.Cu") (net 1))
 (segment (start 147.15 77.315) (end 148.215 76.25) (width 0.2) (layer "F.Cu") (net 9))
 (segment (start 148.215 76.25) (end 149 76.25) (width 0.2) (layer "F.Cu") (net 9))
 (via (at 149 76.25) (size 0.6) (drill 0.3) (layers "F.Cu" "B.Cu") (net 9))
 (segment (start 125 80.75) (end 125.925 81.675) (width 0.2) (layer "B.Cu") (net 9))
 (segment (start 125.925 81.675) (end 127.285 81.675) (width 0.2) (layer "B.Cu") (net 9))
 (segment (start 147.25 66.75) (end 126.5 66.75) (width 0.2) (layer "B.Cu") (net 9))
 (segment (start 149.25 76) (end 149.25 68.75) (width 0.2) (layer "B.Cu") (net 9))
 (segment (start 149.25 68.75) (end 147.25 66.75) (width 0.2) (layer "B.Cu") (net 9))
 (segment (start 125 68.25) (end 125 80.75) (width 0.2) (layer "B.Cu") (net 9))
 (segment (start 149 76.25) (end 149.25 76) (width 0.2) (layer "B.Cu") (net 9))
 (segment (start 126.5 66.75) (end 125 68.25) (width 0.2) (layer "B.Cu") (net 9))
 (segment (start 125 110.75) (end 125 96.66) (width 0.2) (layer "F.Cu") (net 3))
 (segment (start 148.75 81.745) (end 148.75 83.25) (width 0.2) (layer "F.Cu") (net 3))
 (segment (start 152.425 78.07) (end 148.75 81.745) (width 0.2) (layer "F.Cu") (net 3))
 (segment (start 141.5 113.75) (end 128 113.75) (width 0.2) (layer "F.Cu") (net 3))
 (segment (start 125 96.66) (end 127.285 94.375) (width 0.2) (layer "F.Cu") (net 3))
 (segment (start 128 113.75) (end 125 110.75) (width 0.2) (layer "F.Cu") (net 3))
 (via (at 141.5 113.75) (size 0.6) (drill 0.3) (layers "F.Cu" "B.Cu") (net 3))
 (via (at 148.75 83.25) (size 0.6) (drill 0.3) (layers "F.Cu" "B.Cu") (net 3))
 (segment (start 150.351 98.714078) (end 150.351 104.899) (width 0.2) (layer "B.Cu") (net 3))
 (segment (start 148.75 83.25) (end 150.176 84.676) (width 0.2) (layer "B.Cu") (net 3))
 (segment (start 150.176 98.539078) (end 150.351 98.714078) (width 0.2) (layer "B.Cu") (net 3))
 (segment (start 150.176 84.676) (end 150.176 98.539078) (width 0.2) (layer "B.Cu") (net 3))
 (segment (start 150.351 104.899) (end 141.5 113.75) (width 0.2) (layer "B.Cu") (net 3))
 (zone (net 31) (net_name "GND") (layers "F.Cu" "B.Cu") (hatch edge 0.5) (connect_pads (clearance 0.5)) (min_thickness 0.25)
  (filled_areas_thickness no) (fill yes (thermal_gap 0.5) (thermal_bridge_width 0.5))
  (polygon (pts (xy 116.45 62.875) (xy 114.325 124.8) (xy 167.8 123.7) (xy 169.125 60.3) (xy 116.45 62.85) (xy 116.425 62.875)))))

